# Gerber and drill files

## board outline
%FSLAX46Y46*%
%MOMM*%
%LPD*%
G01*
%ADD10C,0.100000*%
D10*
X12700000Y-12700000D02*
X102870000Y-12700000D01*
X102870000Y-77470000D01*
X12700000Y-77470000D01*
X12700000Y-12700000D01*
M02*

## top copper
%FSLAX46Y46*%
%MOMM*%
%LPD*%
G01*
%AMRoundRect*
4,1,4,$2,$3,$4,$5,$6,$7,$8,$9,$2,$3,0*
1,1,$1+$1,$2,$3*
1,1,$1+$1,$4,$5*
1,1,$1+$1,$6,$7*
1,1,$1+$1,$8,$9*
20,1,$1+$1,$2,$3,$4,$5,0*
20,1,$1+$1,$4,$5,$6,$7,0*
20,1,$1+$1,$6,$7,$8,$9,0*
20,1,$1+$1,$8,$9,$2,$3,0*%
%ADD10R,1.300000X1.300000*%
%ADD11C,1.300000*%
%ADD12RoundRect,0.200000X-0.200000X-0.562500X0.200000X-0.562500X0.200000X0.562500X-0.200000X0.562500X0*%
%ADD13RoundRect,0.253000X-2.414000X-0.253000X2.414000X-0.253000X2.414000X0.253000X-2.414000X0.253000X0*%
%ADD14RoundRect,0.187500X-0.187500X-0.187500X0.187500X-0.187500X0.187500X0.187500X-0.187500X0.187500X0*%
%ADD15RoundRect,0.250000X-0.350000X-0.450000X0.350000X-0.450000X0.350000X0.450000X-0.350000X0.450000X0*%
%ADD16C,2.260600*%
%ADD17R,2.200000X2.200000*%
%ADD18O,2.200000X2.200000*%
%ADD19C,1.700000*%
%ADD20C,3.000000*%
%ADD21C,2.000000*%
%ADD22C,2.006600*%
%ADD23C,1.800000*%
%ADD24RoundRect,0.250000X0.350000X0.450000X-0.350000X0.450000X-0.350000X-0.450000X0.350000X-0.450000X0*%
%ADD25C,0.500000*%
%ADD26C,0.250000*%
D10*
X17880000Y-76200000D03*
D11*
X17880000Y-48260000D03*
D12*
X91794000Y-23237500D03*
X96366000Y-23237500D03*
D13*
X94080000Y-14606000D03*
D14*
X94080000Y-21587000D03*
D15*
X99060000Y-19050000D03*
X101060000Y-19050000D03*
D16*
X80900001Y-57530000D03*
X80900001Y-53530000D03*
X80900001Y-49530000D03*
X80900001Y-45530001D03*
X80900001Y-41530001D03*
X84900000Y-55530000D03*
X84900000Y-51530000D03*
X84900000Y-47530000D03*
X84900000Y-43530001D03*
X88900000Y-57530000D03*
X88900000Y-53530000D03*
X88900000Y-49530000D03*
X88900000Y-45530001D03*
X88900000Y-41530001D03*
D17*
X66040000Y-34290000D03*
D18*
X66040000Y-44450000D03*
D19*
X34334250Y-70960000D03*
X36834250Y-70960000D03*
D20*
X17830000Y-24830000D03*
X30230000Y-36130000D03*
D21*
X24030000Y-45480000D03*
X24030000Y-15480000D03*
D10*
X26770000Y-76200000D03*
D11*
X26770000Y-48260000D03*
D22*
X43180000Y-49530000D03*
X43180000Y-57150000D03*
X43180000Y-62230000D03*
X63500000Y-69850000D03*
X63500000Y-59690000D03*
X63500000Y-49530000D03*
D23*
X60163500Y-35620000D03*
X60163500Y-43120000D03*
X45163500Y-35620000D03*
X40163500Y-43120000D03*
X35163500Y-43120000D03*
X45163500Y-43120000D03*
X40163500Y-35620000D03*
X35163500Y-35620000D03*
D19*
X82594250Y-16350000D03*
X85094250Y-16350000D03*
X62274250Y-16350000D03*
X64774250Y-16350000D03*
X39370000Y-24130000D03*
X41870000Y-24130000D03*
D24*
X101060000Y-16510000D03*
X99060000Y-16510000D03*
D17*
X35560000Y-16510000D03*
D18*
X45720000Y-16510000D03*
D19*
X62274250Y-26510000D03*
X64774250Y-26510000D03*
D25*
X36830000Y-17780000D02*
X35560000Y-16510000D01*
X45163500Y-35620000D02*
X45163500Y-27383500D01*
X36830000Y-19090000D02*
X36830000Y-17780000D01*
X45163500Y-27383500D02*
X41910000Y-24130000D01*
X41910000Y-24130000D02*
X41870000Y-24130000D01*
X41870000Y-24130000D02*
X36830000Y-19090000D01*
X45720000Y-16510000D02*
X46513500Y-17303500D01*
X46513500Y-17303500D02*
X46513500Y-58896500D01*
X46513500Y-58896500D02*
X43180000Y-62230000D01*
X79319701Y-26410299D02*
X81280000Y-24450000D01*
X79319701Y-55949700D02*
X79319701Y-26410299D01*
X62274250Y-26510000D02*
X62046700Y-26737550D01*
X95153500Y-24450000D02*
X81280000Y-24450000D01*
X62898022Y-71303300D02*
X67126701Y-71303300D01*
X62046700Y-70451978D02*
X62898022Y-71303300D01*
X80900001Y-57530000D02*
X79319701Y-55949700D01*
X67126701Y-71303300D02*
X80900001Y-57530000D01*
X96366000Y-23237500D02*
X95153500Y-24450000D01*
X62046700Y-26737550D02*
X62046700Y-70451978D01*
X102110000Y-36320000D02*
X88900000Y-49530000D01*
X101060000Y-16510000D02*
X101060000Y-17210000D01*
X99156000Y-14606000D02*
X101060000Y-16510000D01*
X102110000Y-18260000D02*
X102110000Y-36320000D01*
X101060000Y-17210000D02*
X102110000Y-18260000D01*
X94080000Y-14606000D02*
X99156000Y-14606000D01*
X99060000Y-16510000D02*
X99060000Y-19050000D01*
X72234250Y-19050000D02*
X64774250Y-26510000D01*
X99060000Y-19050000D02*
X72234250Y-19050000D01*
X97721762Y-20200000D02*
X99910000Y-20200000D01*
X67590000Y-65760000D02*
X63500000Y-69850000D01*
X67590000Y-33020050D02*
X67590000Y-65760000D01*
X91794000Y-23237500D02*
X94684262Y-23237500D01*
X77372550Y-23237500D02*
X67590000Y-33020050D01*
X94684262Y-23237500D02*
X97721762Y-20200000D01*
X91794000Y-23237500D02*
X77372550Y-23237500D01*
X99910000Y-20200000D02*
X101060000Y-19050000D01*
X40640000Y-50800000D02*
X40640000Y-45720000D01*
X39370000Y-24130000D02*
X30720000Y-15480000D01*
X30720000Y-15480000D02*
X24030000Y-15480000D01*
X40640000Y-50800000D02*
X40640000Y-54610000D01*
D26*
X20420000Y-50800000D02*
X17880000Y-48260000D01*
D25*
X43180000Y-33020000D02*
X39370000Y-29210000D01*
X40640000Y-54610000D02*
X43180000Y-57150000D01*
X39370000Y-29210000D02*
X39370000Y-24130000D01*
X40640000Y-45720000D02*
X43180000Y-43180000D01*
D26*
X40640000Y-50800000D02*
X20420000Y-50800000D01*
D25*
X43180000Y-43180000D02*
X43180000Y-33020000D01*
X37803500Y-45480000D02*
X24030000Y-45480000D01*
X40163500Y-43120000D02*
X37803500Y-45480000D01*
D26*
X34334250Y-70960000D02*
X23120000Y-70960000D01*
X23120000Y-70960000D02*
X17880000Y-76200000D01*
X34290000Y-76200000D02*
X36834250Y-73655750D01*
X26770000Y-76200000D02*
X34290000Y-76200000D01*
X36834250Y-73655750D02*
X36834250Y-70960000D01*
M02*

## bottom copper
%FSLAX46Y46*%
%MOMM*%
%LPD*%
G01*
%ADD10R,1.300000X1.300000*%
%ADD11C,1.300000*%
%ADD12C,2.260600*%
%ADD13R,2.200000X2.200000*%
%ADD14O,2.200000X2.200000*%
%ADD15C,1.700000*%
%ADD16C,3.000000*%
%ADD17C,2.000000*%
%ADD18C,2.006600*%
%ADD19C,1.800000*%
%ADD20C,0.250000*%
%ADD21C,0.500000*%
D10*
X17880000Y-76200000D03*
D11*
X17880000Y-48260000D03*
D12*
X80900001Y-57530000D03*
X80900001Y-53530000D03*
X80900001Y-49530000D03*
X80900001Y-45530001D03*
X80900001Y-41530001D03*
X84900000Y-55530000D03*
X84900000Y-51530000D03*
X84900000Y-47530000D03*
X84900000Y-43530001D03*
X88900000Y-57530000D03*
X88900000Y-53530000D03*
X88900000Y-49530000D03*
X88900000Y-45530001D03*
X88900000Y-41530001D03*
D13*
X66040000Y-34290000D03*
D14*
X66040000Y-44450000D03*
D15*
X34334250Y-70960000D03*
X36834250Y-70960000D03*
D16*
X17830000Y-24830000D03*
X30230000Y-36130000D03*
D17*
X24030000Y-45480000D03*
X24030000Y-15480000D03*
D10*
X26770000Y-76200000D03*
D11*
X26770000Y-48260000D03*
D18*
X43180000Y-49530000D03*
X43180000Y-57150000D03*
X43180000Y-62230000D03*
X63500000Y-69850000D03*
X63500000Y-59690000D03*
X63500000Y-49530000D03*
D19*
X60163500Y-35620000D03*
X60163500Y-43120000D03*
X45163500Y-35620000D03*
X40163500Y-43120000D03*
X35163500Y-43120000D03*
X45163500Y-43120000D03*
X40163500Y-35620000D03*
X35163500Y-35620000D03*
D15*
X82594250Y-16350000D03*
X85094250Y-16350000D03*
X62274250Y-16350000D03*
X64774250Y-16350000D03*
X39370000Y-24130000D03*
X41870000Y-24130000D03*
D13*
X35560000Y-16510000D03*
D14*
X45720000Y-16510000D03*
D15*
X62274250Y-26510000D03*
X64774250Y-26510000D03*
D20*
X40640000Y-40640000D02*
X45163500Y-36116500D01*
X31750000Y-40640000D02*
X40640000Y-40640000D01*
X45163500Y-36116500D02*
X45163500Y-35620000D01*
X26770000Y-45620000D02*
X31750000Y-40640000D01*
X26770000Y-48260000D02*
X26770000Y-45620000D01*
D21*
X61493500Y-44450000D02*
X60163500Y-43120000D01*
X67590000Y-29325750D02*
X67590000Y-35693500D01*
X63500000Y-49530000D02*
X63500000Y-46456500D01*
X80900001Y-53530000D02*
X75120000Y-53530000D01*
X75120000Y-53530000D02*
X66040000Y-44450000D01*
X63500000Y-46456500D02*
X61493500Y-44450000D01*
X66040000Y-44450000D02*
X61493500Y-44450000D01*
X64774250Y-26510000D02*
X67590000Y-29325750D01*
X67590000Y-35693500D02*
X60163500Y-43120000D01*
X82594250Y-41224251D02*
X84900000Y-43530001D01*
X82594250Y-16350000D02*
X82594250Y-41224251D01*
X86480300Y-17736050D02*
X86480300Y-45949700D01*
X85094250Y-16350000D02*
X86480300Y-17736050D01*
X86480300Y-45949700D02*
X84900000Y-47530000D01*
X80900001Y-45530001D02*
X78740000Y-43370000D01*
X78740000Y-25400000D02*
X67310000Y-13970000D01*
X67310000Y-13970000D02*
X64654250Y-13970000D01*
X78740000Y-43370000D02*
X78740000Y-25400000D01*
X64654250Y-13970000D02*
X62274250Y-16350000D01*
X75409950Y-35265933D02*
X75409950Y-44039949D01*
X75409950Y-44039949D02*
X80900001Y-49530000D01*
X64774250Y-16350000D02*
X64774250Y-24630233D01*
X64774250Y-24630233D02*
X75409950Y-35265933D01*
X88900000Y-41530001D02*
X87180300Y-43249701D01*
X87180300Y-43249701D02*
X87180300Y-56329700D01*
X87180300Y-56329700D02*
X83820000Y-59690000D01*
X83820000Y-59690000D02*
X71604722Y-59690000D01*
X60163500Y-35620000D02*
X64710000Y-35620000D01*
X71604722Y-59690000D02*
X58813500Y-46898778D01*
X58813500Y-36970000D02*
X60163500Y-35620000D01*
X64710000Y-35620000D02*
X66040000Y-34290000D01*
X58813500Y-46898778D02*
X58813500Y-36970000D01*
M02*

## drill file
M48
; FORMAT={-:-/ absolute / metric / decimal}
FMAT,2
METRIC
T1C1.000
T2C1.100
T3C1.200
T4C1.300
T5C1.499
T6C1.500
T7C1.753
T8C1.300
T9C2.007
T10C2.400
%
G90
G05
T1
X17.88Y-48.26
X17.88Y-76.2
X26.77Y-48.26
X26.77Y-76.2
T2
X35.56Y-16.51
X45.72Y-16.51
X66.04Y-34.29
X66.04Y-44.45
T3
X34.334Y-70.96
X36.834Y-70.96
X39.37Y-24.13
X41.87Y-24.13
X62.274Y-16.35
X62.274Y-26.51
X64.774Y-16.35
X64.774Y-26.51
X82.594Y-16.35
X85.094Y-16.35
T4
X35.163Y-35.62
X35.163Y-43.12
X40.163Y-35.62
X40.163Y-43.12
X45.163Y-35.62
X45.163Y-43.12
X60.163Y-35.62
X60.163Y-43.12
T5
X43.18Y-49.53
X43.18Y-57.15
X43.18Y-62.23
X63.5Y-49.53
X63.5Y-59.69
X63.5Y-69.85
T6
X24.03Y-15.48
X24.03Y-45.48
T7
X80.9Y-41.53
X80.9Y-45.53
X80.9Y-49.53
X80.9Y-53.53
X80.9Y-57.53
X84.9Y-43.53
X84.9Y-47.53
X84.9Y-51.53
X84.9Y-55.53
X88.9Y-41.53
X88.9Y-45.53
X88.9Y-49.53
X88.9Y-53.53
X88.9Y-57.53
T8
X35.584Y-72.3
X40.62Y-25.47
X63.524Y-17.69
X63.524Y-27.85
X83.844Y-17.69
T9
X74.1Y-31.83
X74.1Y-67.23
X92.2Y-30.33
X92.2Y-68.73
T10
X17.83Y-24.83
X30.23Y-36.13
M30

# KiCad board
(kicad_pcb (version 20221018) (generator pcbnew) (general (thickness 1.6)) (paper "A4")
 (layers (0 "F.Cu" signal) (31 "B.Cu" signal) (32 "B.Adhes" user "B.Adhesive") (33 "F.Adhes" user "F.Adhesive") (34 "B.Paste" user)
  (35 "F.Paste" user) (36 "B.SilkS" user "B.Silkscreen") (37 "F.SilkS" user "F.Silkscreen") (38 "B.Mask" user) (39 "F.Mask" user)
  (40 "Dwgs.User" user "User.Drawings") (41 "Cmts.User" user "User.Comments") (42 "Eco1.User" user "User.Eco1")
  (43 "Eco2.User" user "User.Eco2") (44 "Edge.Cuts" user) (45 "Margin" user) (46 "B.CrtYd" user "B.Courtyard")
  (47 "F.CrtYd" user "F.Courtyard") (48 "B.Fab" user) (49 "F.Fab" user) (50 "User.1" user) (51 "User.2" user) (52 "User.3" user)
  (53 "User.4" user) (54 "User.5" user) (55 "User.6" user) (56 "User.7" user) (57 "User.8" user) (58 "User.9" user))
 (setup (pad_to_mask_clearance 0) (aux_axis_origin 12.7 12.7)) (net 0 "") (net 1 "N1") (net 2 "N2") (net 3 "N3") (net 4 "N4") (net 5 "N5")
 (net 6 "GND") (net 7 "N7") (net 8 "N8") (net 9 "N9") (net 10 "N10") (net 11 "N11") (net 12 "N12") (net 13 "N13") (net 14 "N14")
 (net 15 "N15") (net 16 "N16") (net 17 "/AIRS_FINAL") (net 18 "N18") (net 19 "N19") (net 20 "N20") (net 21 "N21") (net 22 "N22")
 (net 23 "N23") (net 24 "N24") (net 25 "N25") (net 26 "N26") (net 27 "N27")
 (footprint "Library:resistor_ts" (layer "F.Cu") (at 14.1335 72.263 90)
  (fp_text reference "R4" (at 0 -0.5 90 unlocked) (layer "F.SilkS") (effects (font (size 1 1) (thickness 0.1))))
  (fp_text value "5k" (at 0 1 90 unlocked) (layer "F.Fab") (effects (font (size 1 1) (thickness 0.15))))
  (pad "1" thru_hole rect (at -3.937 3.7465 90) (size 1.3 1.3) (drill 1) (layers "*.Cu" "*.Mask") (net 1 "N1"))
  (pad "2" thru_hole circle (at 24.003 3.7465 90) (size 1.3 1.3) (drill 1) (layers "*.Cu" "*.Mask") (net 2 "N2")))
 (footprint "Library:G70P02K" (layer "F.Cu") (at 90.83 15.112)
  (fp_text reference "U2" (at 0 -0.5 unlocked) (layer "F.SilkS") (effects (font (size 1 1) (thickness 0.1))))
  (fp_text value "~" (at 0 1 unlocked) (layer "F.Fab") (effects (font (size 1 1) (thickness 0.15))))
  (pad "1" smd roundrect (at 0.964 8.1255) (size 0.8 1.525) (layers "F.Cu" "F.Paste" "F.Mask") (roundrect_rratio 0.25) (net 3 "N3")
   (thermal_bridge_angle 45))
  (pad "2" smd roundrect (at 5.536 8.1255) (size 0.8 1.525) (layers "F.Cu" "F.Paste" "F.Mask") (roundrect_rratio 0.25) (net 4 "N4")
   (thermal_bridge_angle 45))
  (pad "3" smd roundrect (at 3.25 -0.506) (size 5.334 1.012) (layers "F.Cu" "F.Paste" "F.Mask") (roundrect_rratio 0.25) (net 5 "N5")
   (thermal_bridge_angle 45))
  (pad "4" smd roundrect (at 3.25 6.475) (size 0.75 0.75) (layers "F.Cu" "F.Paste" "F.Mask") (roundrect_rratio 0.25)
   (thermal_bridge_angle 45)))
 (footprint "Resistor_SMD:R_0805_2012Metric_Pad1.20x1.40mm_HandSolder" (layer "F.Cu") (at 100.06 19.05)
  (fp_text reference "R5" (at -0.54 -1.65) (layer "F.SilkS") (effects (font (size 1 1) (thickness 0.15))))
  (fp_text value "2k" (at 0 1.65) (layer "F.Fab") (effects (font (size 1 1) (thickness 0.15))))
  (pad "1" smd roundrect (at -1 0) (size 1.2 1.4) (layers "F.Cu" "F.Paste" "F.Mask") (roundrect_rratio 0.2083333333) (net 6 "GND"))
  (pad "2" smd roundrect (at 1 0) (size 1.2 1.4) (layers "F.Cu" "F.Paste" "F.Mask") (roundrect_rratio 0.2083333333) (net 3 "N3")))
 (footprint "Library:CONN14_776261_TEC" (layer "F.Cu") (at 88.9 41.530001 90)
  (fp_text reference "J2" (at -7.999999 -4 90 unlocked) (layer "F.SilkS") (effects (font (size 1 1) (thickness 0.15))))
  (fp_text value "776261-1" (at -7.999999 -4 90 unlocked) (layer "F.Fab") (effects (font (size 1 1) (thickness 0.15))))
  (pad "" np_thru_hole circle (at -27.199999 3.300001 90) (size 2.0066 2.0066) (drill 2.0066) (layers "*.Cu" "*.Mask"))
  (pad "" np_thru_hole circle (at -25.700003 -14.799999 90) (size 2.0066 2.0066) (drill 2.0066) (layers "*.Cu" "*.Mask"))
  (pad "" np_thru_hole circle (at 9.700004 -14.799999 90) (size 2.0066 2.0066) (drill 2.0066) (layers "*.Cu" "*.Mask"))
  (pad "" np_thru_hole circle (at 11.200001 3.300001 90) (size 2.0066 2.0066) (drill 2.0066) (layers "*.Cu" "*.Mask"))
  (pad "1" thru_hole circle (at -15.999999 -7.999999 90) (size 2.2606 2.2606) (drill 1.7526) (layers "*.Cu" "*.Mask") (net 4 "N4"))
  (pad "2" thru_hole circle (at -11.999999 -7.999999 90) (size 2.2606 2.2606) (drill 1.7526) (layers "*.Cu" "*.Mask") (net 6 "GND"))
  (pad "3" thru_hole circle (at -7.999999 -7.999999 90) (size 2.2606 2.2606) (drill 1.7526) (layers "*.Cu" "*.Mask") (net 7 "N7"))
  (pad "4" thru_hole circle (at -4 -7.999999 90) (size 2.2606 2.2606) (drill 1.7526) (layers "*.Cu" "*.Mask") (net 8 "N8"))
  (pad "5" thru_hole circle (at 0 -7.999999 90) (size 2.2606 2.2606) (drill 1.7526) (layers "*.Cu" "*.Mask") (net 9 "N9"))
  (pad "6" thru_hole circle (at -13.999999 -4 90) (size 2.2606 2.2606) (drill 1.7526) (layers "*.Cu" "*.Mask") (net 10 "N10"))
  (pad "7" thru_hole circle (at -9.999999 -4 90) (size 2.2606 2.2606) (drill 1.7526) (layers "*.Cu" "*.Mask") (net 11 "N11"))
  (pad "8" thru_hole circle (at -5.999999 -4 90) (size 2.2606 2.2606) (drill 1.7526) (layers "*.Cu" "*.Mask") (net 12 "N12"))
  (pad "9" thru_hole circle (at -2 -4 90) (size 2.2606 2.2606) (drill 1.7526) (layers "*.Cu" "*.Mask") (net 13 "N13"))
  (pad "10" thru_hole circle (at -15.999999 0 90) (size 2.2606 2.2606) (drill 1.7526) (layers "*.Cu" "*.Mask") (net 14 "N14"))
  (pad "11" thru_hole circle (at -11.999999 0 90) (size 2.2606 2.2606) (drill 1.7526) (layers "*.Cu" "*.Mask") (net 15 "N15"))
  (pad "12" thru_hole circle (at -7.999999 0 90) (size 2.2606 2.2606) (drill 1.7526) (layers "*.Cu" "*.Mask") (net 5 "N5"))
  (pad "13" thru_hole circle (at -4 0 90) (size 2.2606 2.2606) (drill 1.7526) (layers "*.Cu" "*.Mask") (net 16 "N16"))
  (pad "14" thru_hole circle (at 0 0 90) (size 2.2606 2.2606) (drill 1.7526) (layers "*.Cu" "*.Mask") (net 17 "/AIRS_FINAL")))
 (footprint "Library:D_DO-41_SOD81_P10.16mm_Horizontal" (layer "F.Cu") (at 66.04 34.29 -90)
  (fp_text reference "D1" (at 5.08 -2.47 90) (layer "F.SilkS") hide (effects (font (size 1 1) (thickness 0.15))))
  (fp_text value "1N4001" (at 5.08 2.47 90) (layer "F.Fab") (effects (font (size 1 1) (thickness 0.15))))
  (pad "1" thru_hole rect (at 0 0 270) (size 2.2 2.2) (drill 1.1) (layers "*.Cu" "*.Mask") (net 17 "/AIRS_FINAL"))
  (pad "2" thru_hole oval (at 10.16 0 270) (size 2.2 2.2) (drill 1.1) (layers "*.Cu" "*.Mask") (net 6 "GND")))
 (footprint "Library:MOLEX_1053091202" (layer "F.Cu") (at 34.33425 70.96)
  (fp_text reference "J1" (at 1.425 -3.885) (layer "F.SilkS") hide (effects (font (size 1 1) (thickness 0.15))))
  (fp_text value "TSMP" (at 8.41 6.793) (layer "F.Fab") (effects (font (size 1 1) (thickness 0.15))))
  (pad "" np_thru_hole circle (at 1.25 1.34) (size 1.3 1.3) (drill 1.3) (layers "*.Cu" "*.Mask"))
  (pad "1" thru_hole circle (at 0 0) (size 1.7 1.7) (drill 1.2) (layers "*.Cu") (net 1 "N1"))
  (pad "2" thru_hole circle (at 2.5 0) (size 1.7 1.7) (drill 1.2) (layers "*.Cu") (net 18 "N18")))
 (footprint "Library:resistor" (layer "F.Cu") (at 32.53 21.98 -90)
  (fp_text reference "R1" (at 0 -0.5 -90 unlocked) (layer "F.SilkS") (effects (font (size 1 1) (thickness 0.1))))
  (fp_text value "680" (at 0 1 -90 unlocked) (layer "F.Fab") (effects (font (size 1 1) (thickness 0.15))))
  (pad "" np_thru_hole circle (at 2.85 14.7 270) (size 3 3) (drill 2.4) (layers "F&B.Cu" "*.Mask"))
  (pad "" np_thru_hole circle (at 14.15 2.3 270) (size 3 3) (drill 2.4) (layers "F&B.Cu" "*.Mask"))
  (pad "1" thru_hole circle (at 23.5 8.5 270) (size 2 2) (drill 1.5) (layers "*.Cu" "*.Mask") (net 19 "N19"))
  (pad "2" thru_hole circle (at -6.5 8.5 270) (size 2 2) (drill 1.5) (layers "*.Cu" "*.Mask") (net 2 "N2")))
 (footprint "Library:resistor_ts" (layer "F.Cu") (at 23.0235 72.263 90)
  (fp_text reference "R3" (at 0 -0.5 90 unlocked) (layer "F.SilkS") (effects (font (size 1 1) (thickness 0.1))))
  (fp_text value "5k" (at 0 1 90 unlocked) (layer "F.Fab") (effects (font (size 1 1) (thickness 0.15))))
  (pad "1" thru_hole rect (at -3.937 3.7465 90) (size 1.3 1.3) (drill 1) (layers "*.Cu" "*.Mask") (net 18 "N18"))
  (pad "2" thru_hole circle (at 24.003 3.7465 90) (size 1.3 1.3) (drill 1) (layers "*.Cu" "*.Mask") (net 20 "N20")))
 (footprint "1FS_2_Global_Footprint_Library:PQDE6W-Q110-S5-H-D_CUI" (layer "F.Cu") (at 43.18 49.53)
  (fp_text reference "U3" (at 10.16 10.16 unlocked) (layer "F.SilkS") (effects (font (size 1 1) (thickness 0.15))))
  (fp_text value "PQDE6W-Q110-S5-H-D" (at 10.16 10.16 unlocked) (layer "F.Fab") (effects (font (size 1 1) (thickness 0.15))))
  (pad "1" thru_hole circle (at 0 0) (size 2.0066 2.0066) (drill 1.4986) (layers "*.Cu" "*.Mask") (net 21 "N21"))
  (pad "2" thru_hole circle (at 0 7.62) (size 2.0066 2.0066) (drill 1.4986) (layers "*.Cu" "*.Mask") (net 2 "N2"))
  (pad "3" thru_hole circle (at 0 12.7) (size 2.0066 2.0066) (drill 1.4986) (layers "*.Cu" "*.Mask") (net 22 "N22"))
  (pad "4" thru_hole circle (at 20.32 20.32) (size 2.0066 2.0066) (drill 1.4986) (layers "*.Cu" "*.Mask") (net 3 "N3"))
  (pad "5" thru_hole circle (at 20.32 10.16) (size 2.0066 2.0066) (drill 1.4986) (layers "*.Cu" "*.Mask") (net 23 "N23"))
  (pad "6" thru_hole circle (at 20.32 0) (size 2.0066 2.0066) (drill 1.4986) (layers "*.Cu" "*.Mask") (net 6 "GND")))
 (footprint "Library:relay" (layer "F.Cu") (at 62.6635 33.12 -90)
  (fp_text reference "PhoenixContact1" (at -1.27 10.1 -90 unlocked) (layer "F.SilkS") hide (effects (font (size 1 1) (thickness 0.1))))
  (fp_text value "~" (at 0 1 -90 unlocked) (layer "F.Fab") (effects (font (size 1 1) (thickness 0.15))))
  (pad "1" thru_hole circle (at 2.5 2.5 270) (size 1.8 1.8) (drill 1.3) (layers "*.Cu" "*.Mask") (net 17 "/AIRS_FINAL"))
  (pad "2" thru_hole circle (at 10 2.5 270) (size 1.8 1.8) (drill 1.3) (layers "*.Cu" "*.Mask") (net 6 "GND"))
  (pad "3" thru_hole circle (at 2.5 17.5 270) (size 1.8 1.8) (drill 1.3) (layers "*.Cu" "*.Mask") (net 20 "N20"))
  (pad "4" thru_hole circle (at 10 22.5 270) (size 1.8 1.8) (drill 1.3) (layers "*.Cu" "*.Mask") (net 19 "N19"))
  (pad "5" thru_hole circle (at 10 27.5 270) (size 1.8 1.8) (drill 1.3) (layers "*.Cu" "*.Mask") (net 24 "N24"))
  (pad "6" thru_hole circle (at 10 17.5 270) (size 1.8 1.8) (drill 1.3) (layers "*.Cu" "*.Mask") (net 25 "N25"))
  (pad "7" thru_hole circle (at 2.5 22.5 270) (size 1.8 1.8) (drill 1.3) (layers "*.Cu" "*.Mask") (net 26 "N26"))
  (pad "8" thru_hole circle (at 2.5 27.5 270) (size 1.8 1.8) (drill 1.3) (layers "*.Cu" "*.Mask") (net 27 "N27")))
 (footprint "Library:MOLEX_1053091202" (layer "F.Cu") (at 82.59425 16.35)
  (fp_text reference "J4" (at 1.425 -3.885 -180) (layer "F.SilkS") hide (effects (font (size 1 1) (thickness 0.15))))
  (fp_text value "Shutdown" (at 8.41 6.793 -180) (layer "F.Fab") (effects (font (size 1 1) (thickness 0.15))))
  (pad "" np_thru_hole circle (at 1.25 1.34) (size 1.3 1.3) (drill 1.3) (layers "*.Cu" "*.Mask"))
  (pad "1" thru_hole circle (at 0 0) (size 1.7 1.7) (drill 1.2) (layers "*.Cu") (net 13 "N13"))
  (pad "2" thru_hole circle (at 2.5 0) (size 1.7 1.7) (drill 1.2) (layers "*.Cu") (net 12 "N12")))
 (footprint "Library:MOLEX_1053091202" (layer "F.Cu") (at 62.27425 16.35)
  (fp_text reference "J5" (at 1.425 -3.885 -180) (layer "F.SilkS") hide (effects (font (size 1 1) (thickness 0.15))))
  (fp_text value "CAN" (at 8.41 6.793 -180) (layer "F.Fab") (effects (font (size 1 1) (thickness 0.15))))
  (pad "" np_thru_hole circle (at 1.25 1.34) (size 1.3 1.3) (drill 1.3) (layers "*.Cu" "*.Mask"))
  (pad "1" thru_hole circle (at 0 0) (size 1.7 1.7) (drill 1.2) (layers "*.Cu") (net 8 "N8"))
  (pad "2" thru_hole circle (at 2.5 0) (size 1.7 1.7) (drill 1.2) (layers "*.Cu") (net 7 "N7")))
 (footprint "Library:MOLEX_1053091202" (layer "F.Cu") (at 39.37 24.13)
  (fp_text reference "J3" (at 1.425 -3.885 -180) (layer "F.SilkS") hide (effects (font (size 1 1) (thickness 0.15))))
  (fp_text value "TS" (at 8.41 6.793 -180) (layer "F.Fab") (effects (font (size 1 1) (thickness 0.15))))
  (pad "" np_thru_hole circle (at 1.25 1.34) (size 1.3 1.3) (drill 1.3) (layers "*.Cu" "*.Mask"))
  (pad "1" thru_hole circle (at 0 0) (size 1.7 1.7) (drill 1.2) (layers "*.Cu") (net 2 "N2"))
  (pad "2" thru_hole circle (at 2.5 0) (size 1.7 1.7) (drill 1.2) (layers "*.Cu") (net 20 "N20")))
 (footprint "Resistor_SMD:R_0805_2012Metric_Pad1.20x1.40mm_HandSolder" (layer "F.Cu") (at 100.06 16.51 180)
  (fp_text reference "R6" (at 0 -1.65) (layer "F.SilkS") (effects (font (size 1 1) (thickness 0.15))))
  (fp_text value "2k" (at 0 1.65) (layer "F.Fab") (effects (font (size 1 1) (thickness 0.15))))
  (pad "1" smd roundrect (at -1 0 180) (size 1.2 1.4) (layers "F.Cu" "F.Paste" "F.Mask") (roundrect_rratio 0.2083333333) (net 5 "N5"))
  (pad "2" smd roundrect (at 1 0 180) (size 1.2 1.4) (layers "F.Cu" "F.Paste" "F.Mask") (roundrect_rratio 0.2083333333) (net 6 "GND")))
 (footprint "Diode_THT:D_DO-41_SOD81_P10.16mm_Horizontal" (layer "F.Cu") (at 35.56 16.51)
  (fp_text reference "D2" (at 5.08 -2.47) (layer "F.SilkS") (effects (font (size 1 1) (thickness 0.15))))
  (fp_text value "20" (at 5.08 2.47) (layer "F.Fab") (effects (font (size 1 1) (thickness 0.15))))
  (pad "1" thru_hole rect (at 0 0) (size 2.2 2.2) (drill 1.1) (layers "*.Cu" "*.Mask") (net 20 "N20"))
  (pad "2" thru_hole oval (at 10.16 0) (size 2.2 2.2) (drill 1.1) (layers "*.Cu" "*.Mask") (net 22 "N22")))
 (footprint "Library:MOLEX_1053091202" (layer "F.Cu") (at 62.27425 26.51)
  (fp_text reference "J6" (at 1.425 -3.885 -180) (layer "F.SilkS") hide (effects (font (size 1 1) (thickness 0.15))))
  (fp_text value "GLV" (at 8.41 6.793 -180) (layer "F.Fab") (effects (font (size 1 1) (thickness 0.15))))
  (pad "" np_thru_hole circle (at 1.25 1.34) (size 1.3 1.3) (drill 1.3) (layers "*.Cu" "*.Mask"))
  (pad "1" thru_hole circle (at 0 0) (size 1.7 1.7) (drill 1.2) (layers "*.Cu") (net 4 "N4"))
  (pad "2" thru_hole circle (at 2.5 0) (size 1.7 1.7) (drill 1.2) (layers "*.Cu") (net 6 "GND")))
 (gr_rect (start 12.7 12.7) (end 102.87 77.47) (stroke (width 0.1) (type default)) (fill none) (layer "Edge.Cuts"))
 (segment (start 36.83 17.78) (end 35.56 16.51) (width 0.5) (layer "F.Cu") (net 20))
 (segment (start 45.1635 35.62) (end 45.1635 27.3835) (width 0.5) (layer "F.Cu") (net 20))
 (segment (start 36.83 19.09) (end 36.83 17.78) (width 0.5) (layer "F.Cu") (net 20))
 (segment (start 45.1635 27.3835) (end 41.91 24.13) (width 0.5) (layer "F.Cu") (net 20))
 (segment (start 41.91 24.13) (end 41.87 24.13) (width 0.5) (layer "F.Cu") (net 20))
 (segment (start 41.87 24.13) (end 36.83 19.09) (width 0.5) (layer "F.Cu") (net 20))
 (segment (start 40.64 40.64) (end 45.1635 36.1165) (width 0.25) (layer "B.Cu") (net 20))
 (segment (start 31.75 40.64) (end 40.64 40.64) (width 0.25) (layer "B.Cu") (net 20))
 (segment (start 45.1635 36.1165) (end 45.1635 35.62) (width 0.25) (layer "B.Cu") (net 20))
 (segment (start 26.77 45.62) (end 31.75 40.64) (width 0.25) (layer "B.Cu") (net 20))
 (segment (start 26.77 48.26) (end 26.77 45.62) (width 0.25) (layer "B.Cu") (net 20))
 (segment (start 45.72 16.51) (end 46.5135 17.3035) (width 0.5) (layer "F.Cu") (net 22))
 (segment (start 46.5135 17.3035) (end 46.5135 58.8965) (width 0.5) (layer "F.Cu") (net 22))
 (segment (start 46.5135 58.8965) (end 43.18 62.23) (width 0.5) (layer "F.Cu") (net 22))
 (segment (start 79.319701 26.410299) (end 81.28 24.45) (width 0.5) (layer "F.Cu") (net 4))
 (segment (start 79.319701 55.9497) (end 79.319701 26.410299) (width 0.5) (layer "F.Cu") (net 4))
 (segment (start 62.27425 26.51) (end 62.0467 26.73755) (width 0.5) (layer "F.Cu") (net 4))
 (segment (start 95.1535 24.45) (end 81.28 24.45) (width 0.5) (layer "F.Cu") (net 4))
 (segment (start 62.898022 71.3033) (end 67.126701 71.3033) (width 0.5) (layer "F.Cu") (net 4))
 (segment (start 62.0467 70.451978) (end 62.898022 71.3033) (width 0.5) (layer "F.Cu") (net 4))
 (segment (start 80.900001 57.53) (end 79.319701 55.9497) (width 0.5) (layer "F.Cu") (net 4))
 (segment (start 67.126701 71.3033) (end 80.900001 57.53) (width 0.5) (layer "F.Cu") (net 4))
 (segment (start 96.366 23.2375) (end 95.1535 24.45) (width 0.5) (layer "F.Cu") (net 4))
 (segment (start 62.0467 26.73755) (end 62.0467 70.451978) (width 0.5) (layer "F.Cu") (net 4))
 (segment (start 102.11 36.32) (end 88.9 49.53) (width 0.5) (layer "F.Cu") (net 5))
 (segment (start 101.06 16.51) (end 101.06 17.21) (width 0.5) (layer "F.Cu") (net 5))
 (segment (start 99.156 14.606) (end 101.06 16.51) (width 0.5) (layer "F.Cu") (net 5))
 (segment (start 102.11 18.26) (end 102.11 36.32) (width 0.5) (layer "F.Cu") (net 5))
 (segment (start 101.06 17.21) (end 102.11 18.26) (width 0.5) (layer "F.Cu") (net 5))
 (segment (start 94.08 14.606) (end 99.156 14.606) (width 0.5) (layer "F.Cu") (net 5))
 (segment (start 99.06 16.51) (end 99.06 19.05) (width 0.5) (layer "F.Cu") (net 6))
 (segment (start 72.23425 19.05) (end 64.77425 26.51) (width 0.5) (layer "F.Cu") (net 6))
 (segment (start 99.06 19.05) (end 72.23425 19.05) (width 0.5) (layer "F.Cu") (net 6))
 (segment (start 61.4935 44.45) (end 60.1635 43.12) (width 0.5) (layer "B.Cu") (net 6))
 (segment (start 67.59 29.32575) (end 67.59 35.6935) (width 0.5) (layer "B.Cu") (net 6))
 (segment (start 63.5 49.53) (end 63.5 46.4565) (width 0.5) (layer "B.Cu") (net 6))
 (segment (start 80.900001 53.53) (end 75.12 53.53) (width 0.5) (layer "B.Cu") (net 6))
 (segment (start 75.12 53.53) (end 66.04 44.45) (width 0.5) (layer "B.Cu") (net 6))
 (segment (start 63.5 46.4565) (end 61.4935 44.45) (width 0.5) (layer "B.Cu") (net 6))
 (segment (start 66.04 44.45) (end 61.4935 44.45) (width 0.5) (layer "B.Cu") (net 6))
 (segment (start 64.77425 26.51) (end 67.59 29.32575) (width 0.5) (layer "B.Cu") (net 6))
 (segment (start 67.59 35.6935) (end 60.1635 43.12) (width 0.5) (layer "B.Cu") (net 6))
 (segment (start 97.721762 20.2) (end 99.91 20.2) (width 0.5) (layer "F.Cu") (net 3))
 (segment (start 67.59 65.76) (end 63.5 69.85) (width 0.5) (layer "F.Cu") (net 3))
 (segment (start 67.59 33.02005) (end 67.59 65.76) (width 0.5) (layer "F.Cu") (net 3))
 (segment (start 91.794 23.2375) (end 94.684262 23.2375) (width 0.5) (layer "F.Cu") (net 3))
 (segment (start 77.37255 23.2375) (end 67.59 33.02005) (width 0.5) (layer "F.Cu") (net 3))
 (segment (start 94.684262 23.2375) (end 97.721762 20.2) (width 0.5) (layer "F.Cu") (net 3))
 (segment (start 91.794 23.2375) (end 77.37255 23.2375) (width 0.5) (layer "F.Cu") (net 3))
 (segment (start 99.91 20.2) (end 101.06 19.05) (width 0.5) (layer "F.Cu") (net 3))
 (segment (start 40.64 50.8) (end 40.64 45.72) (width 0.5) (layer "F.Cu") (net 2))
 (segment (start 39.37 24.13) (end 30.72 15.48) (width 0.5) (layer "F.Cu") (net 2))
 (segment (start 30.72 15.48) (end 24.03 15.48) (width 0.5) (layer "F.Cu") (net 2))
 (segment (start 40.64 50.8) (end 40.64 54.61) (width 0.5) (layer "F.Cu") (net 2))
 (segment (start 20.42 50.8) (end 17.88 48.26) (width 0.25) (layer "F.Cu") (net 2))
 (segment (start 43.18 33.02) (end 39.37 29.21) (width 0.5) (layer "F.Cu") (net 2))
 (segment (start 40.64 54.61) (end 43.18 57.15) (width 0.5) (layer "F.Cu") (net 2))
 (segment (start 39.37 29.21) (end 39.37 24.13) (width 0.5) (layer "F.Cu") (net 2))
 (segment (start 40.64 45.72) (end 43.18 43.18) (width 0.5) (layer "F.Cu") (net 2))
 (segment (start 40.64 50.8) (end 20.42 50.8) (width 0.25) (layer "F.Cu") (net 2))
 (segment (start 43.18 43.18) (end 43.18 33.02) (width 0.5) (layer "F.Cu") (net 2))
 (segment (start 82.59425 41.224251) (end 84.9 43.530001) (width 0.5) (layer "B.Cu") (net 13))
 (segment (start 82.59425 16.35) (end 82.59425 41.224251) (width 0.5) (layer "B.Cu") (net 13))
 (segment (start 86.4803 17.73605) (end 86.4803 45.9497) (width 0.5) (layer "B.Cu") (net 12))
 (segment (start 85.09425 16.35) (end 86.4803 17.73605) (width 0.5) (layer "B.Cu") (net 12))
 (segment (start 86.4803 45.9497) (end 84.9 47.53) (width 0.5) (layer "B.Cu") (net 12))
 (segment (start 80.900001 45.530001) (end 78.74 43.37) (width 0.5) (layer "B.Cu") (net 8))
 (segment (start 78.74 25.4) (end 67.31 13.97) (width 0.5) (layer "B.Cu") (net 8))
 (segment (start 67.31 13.97) (end 64.65425 13.97) (width 0.5) (layer "B.Cu") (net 8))
 (segment (start 78.74 43.37) (end 78.74 25.4) (width 0.5) (layer "B.Cu") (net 8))
 (segment (start 64.65425 13.97) (end 62.27425 16.35) (width 0.5) (layer "B.Cu") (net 8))
 (segment (start 75.40995 35.265933) (end 75.40995 44.039949) (width 0.5) (layer "B.Cu") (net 7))
 (segment (start 75.40995 44.039949) (end 80.900001 49.53) (width 0.5) (layer "B.Cu") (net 7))
 (segment (start 64.77425 16.35) (end 64.77425 24.630233) (width 0.5) (layer "B.Cu") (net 7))
 (segment (start 64.77425 24.630233) (end 75.40995 35.265933) (width 0.5) (layer "B.Cu") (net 7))
 (segment (start 88.9 41.530001) (end 87.1803 43.249701) (width 0.5) (layer "B.Cu") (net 17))
 (segment (start 87.1803 43.249701) (end 87.1803 56.3297) (width 0.5) (layer "B.Cu") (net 17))
 (segment (start 87.1803 56.3297) (end 83.82 59.69) (width 0.5) (layer "B.Cu") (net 17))
 (segment (start 83.82 59.69) (end 71.604722 59.69) (width 0.5) (layer "B.Cu") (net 17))
 (segment (start 60.1635 35.62) (end 64.71 35.62) (width 0.5) (layer "B.Cu") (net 17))
 (segment (start 71.604722 59.69) (end 58.8135 46.898778) (width 0.5) (layer "B.Cu") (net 17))
 (segment (start 58.8135 36.97) (end 60.1635 35.62) (width 0.5) (layer "B.Cu") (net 17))
 (segment (start 64.71 35.62) (end 66.04 34.29) (width 0.5) (layer "B.Cu") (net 17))
 (segment (start 58.8135 46.898778) (end 58.8135 36.97) (width 0.5) (layer "B.Cu") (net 17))
 (segment (start 37.8035 45.48) (end 24.03 45.48) (width 0.5) (layer "F.Cu") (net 19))
 (segment (start 40.1635 43.12) (end 37.8035 45.48) (width 0.5) (layer "F.Cu") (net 19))
 (segment (start 34.33425 70.96) (end 23.12 70.96) (width 0.25) (layer "F.Cu") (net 1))
 (segment (start 23.12 70.96) (end 17.88 76.2) (width 0.25) (layer "F.Cu") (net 1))
 (segment (start 34.29 76.2) (end 36.83425 73.65575) (width 0.25) (layer "F.Cu") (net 18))
 (segment (start 26.77 76.2) (end 34.29 76.2) (width 0.25) (layer "F.Cu") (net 18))
 (segment (start 36.83425 73.65575) (end 36.83425 70.96) (width 0.25) (layer "F.Cu") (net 18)))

